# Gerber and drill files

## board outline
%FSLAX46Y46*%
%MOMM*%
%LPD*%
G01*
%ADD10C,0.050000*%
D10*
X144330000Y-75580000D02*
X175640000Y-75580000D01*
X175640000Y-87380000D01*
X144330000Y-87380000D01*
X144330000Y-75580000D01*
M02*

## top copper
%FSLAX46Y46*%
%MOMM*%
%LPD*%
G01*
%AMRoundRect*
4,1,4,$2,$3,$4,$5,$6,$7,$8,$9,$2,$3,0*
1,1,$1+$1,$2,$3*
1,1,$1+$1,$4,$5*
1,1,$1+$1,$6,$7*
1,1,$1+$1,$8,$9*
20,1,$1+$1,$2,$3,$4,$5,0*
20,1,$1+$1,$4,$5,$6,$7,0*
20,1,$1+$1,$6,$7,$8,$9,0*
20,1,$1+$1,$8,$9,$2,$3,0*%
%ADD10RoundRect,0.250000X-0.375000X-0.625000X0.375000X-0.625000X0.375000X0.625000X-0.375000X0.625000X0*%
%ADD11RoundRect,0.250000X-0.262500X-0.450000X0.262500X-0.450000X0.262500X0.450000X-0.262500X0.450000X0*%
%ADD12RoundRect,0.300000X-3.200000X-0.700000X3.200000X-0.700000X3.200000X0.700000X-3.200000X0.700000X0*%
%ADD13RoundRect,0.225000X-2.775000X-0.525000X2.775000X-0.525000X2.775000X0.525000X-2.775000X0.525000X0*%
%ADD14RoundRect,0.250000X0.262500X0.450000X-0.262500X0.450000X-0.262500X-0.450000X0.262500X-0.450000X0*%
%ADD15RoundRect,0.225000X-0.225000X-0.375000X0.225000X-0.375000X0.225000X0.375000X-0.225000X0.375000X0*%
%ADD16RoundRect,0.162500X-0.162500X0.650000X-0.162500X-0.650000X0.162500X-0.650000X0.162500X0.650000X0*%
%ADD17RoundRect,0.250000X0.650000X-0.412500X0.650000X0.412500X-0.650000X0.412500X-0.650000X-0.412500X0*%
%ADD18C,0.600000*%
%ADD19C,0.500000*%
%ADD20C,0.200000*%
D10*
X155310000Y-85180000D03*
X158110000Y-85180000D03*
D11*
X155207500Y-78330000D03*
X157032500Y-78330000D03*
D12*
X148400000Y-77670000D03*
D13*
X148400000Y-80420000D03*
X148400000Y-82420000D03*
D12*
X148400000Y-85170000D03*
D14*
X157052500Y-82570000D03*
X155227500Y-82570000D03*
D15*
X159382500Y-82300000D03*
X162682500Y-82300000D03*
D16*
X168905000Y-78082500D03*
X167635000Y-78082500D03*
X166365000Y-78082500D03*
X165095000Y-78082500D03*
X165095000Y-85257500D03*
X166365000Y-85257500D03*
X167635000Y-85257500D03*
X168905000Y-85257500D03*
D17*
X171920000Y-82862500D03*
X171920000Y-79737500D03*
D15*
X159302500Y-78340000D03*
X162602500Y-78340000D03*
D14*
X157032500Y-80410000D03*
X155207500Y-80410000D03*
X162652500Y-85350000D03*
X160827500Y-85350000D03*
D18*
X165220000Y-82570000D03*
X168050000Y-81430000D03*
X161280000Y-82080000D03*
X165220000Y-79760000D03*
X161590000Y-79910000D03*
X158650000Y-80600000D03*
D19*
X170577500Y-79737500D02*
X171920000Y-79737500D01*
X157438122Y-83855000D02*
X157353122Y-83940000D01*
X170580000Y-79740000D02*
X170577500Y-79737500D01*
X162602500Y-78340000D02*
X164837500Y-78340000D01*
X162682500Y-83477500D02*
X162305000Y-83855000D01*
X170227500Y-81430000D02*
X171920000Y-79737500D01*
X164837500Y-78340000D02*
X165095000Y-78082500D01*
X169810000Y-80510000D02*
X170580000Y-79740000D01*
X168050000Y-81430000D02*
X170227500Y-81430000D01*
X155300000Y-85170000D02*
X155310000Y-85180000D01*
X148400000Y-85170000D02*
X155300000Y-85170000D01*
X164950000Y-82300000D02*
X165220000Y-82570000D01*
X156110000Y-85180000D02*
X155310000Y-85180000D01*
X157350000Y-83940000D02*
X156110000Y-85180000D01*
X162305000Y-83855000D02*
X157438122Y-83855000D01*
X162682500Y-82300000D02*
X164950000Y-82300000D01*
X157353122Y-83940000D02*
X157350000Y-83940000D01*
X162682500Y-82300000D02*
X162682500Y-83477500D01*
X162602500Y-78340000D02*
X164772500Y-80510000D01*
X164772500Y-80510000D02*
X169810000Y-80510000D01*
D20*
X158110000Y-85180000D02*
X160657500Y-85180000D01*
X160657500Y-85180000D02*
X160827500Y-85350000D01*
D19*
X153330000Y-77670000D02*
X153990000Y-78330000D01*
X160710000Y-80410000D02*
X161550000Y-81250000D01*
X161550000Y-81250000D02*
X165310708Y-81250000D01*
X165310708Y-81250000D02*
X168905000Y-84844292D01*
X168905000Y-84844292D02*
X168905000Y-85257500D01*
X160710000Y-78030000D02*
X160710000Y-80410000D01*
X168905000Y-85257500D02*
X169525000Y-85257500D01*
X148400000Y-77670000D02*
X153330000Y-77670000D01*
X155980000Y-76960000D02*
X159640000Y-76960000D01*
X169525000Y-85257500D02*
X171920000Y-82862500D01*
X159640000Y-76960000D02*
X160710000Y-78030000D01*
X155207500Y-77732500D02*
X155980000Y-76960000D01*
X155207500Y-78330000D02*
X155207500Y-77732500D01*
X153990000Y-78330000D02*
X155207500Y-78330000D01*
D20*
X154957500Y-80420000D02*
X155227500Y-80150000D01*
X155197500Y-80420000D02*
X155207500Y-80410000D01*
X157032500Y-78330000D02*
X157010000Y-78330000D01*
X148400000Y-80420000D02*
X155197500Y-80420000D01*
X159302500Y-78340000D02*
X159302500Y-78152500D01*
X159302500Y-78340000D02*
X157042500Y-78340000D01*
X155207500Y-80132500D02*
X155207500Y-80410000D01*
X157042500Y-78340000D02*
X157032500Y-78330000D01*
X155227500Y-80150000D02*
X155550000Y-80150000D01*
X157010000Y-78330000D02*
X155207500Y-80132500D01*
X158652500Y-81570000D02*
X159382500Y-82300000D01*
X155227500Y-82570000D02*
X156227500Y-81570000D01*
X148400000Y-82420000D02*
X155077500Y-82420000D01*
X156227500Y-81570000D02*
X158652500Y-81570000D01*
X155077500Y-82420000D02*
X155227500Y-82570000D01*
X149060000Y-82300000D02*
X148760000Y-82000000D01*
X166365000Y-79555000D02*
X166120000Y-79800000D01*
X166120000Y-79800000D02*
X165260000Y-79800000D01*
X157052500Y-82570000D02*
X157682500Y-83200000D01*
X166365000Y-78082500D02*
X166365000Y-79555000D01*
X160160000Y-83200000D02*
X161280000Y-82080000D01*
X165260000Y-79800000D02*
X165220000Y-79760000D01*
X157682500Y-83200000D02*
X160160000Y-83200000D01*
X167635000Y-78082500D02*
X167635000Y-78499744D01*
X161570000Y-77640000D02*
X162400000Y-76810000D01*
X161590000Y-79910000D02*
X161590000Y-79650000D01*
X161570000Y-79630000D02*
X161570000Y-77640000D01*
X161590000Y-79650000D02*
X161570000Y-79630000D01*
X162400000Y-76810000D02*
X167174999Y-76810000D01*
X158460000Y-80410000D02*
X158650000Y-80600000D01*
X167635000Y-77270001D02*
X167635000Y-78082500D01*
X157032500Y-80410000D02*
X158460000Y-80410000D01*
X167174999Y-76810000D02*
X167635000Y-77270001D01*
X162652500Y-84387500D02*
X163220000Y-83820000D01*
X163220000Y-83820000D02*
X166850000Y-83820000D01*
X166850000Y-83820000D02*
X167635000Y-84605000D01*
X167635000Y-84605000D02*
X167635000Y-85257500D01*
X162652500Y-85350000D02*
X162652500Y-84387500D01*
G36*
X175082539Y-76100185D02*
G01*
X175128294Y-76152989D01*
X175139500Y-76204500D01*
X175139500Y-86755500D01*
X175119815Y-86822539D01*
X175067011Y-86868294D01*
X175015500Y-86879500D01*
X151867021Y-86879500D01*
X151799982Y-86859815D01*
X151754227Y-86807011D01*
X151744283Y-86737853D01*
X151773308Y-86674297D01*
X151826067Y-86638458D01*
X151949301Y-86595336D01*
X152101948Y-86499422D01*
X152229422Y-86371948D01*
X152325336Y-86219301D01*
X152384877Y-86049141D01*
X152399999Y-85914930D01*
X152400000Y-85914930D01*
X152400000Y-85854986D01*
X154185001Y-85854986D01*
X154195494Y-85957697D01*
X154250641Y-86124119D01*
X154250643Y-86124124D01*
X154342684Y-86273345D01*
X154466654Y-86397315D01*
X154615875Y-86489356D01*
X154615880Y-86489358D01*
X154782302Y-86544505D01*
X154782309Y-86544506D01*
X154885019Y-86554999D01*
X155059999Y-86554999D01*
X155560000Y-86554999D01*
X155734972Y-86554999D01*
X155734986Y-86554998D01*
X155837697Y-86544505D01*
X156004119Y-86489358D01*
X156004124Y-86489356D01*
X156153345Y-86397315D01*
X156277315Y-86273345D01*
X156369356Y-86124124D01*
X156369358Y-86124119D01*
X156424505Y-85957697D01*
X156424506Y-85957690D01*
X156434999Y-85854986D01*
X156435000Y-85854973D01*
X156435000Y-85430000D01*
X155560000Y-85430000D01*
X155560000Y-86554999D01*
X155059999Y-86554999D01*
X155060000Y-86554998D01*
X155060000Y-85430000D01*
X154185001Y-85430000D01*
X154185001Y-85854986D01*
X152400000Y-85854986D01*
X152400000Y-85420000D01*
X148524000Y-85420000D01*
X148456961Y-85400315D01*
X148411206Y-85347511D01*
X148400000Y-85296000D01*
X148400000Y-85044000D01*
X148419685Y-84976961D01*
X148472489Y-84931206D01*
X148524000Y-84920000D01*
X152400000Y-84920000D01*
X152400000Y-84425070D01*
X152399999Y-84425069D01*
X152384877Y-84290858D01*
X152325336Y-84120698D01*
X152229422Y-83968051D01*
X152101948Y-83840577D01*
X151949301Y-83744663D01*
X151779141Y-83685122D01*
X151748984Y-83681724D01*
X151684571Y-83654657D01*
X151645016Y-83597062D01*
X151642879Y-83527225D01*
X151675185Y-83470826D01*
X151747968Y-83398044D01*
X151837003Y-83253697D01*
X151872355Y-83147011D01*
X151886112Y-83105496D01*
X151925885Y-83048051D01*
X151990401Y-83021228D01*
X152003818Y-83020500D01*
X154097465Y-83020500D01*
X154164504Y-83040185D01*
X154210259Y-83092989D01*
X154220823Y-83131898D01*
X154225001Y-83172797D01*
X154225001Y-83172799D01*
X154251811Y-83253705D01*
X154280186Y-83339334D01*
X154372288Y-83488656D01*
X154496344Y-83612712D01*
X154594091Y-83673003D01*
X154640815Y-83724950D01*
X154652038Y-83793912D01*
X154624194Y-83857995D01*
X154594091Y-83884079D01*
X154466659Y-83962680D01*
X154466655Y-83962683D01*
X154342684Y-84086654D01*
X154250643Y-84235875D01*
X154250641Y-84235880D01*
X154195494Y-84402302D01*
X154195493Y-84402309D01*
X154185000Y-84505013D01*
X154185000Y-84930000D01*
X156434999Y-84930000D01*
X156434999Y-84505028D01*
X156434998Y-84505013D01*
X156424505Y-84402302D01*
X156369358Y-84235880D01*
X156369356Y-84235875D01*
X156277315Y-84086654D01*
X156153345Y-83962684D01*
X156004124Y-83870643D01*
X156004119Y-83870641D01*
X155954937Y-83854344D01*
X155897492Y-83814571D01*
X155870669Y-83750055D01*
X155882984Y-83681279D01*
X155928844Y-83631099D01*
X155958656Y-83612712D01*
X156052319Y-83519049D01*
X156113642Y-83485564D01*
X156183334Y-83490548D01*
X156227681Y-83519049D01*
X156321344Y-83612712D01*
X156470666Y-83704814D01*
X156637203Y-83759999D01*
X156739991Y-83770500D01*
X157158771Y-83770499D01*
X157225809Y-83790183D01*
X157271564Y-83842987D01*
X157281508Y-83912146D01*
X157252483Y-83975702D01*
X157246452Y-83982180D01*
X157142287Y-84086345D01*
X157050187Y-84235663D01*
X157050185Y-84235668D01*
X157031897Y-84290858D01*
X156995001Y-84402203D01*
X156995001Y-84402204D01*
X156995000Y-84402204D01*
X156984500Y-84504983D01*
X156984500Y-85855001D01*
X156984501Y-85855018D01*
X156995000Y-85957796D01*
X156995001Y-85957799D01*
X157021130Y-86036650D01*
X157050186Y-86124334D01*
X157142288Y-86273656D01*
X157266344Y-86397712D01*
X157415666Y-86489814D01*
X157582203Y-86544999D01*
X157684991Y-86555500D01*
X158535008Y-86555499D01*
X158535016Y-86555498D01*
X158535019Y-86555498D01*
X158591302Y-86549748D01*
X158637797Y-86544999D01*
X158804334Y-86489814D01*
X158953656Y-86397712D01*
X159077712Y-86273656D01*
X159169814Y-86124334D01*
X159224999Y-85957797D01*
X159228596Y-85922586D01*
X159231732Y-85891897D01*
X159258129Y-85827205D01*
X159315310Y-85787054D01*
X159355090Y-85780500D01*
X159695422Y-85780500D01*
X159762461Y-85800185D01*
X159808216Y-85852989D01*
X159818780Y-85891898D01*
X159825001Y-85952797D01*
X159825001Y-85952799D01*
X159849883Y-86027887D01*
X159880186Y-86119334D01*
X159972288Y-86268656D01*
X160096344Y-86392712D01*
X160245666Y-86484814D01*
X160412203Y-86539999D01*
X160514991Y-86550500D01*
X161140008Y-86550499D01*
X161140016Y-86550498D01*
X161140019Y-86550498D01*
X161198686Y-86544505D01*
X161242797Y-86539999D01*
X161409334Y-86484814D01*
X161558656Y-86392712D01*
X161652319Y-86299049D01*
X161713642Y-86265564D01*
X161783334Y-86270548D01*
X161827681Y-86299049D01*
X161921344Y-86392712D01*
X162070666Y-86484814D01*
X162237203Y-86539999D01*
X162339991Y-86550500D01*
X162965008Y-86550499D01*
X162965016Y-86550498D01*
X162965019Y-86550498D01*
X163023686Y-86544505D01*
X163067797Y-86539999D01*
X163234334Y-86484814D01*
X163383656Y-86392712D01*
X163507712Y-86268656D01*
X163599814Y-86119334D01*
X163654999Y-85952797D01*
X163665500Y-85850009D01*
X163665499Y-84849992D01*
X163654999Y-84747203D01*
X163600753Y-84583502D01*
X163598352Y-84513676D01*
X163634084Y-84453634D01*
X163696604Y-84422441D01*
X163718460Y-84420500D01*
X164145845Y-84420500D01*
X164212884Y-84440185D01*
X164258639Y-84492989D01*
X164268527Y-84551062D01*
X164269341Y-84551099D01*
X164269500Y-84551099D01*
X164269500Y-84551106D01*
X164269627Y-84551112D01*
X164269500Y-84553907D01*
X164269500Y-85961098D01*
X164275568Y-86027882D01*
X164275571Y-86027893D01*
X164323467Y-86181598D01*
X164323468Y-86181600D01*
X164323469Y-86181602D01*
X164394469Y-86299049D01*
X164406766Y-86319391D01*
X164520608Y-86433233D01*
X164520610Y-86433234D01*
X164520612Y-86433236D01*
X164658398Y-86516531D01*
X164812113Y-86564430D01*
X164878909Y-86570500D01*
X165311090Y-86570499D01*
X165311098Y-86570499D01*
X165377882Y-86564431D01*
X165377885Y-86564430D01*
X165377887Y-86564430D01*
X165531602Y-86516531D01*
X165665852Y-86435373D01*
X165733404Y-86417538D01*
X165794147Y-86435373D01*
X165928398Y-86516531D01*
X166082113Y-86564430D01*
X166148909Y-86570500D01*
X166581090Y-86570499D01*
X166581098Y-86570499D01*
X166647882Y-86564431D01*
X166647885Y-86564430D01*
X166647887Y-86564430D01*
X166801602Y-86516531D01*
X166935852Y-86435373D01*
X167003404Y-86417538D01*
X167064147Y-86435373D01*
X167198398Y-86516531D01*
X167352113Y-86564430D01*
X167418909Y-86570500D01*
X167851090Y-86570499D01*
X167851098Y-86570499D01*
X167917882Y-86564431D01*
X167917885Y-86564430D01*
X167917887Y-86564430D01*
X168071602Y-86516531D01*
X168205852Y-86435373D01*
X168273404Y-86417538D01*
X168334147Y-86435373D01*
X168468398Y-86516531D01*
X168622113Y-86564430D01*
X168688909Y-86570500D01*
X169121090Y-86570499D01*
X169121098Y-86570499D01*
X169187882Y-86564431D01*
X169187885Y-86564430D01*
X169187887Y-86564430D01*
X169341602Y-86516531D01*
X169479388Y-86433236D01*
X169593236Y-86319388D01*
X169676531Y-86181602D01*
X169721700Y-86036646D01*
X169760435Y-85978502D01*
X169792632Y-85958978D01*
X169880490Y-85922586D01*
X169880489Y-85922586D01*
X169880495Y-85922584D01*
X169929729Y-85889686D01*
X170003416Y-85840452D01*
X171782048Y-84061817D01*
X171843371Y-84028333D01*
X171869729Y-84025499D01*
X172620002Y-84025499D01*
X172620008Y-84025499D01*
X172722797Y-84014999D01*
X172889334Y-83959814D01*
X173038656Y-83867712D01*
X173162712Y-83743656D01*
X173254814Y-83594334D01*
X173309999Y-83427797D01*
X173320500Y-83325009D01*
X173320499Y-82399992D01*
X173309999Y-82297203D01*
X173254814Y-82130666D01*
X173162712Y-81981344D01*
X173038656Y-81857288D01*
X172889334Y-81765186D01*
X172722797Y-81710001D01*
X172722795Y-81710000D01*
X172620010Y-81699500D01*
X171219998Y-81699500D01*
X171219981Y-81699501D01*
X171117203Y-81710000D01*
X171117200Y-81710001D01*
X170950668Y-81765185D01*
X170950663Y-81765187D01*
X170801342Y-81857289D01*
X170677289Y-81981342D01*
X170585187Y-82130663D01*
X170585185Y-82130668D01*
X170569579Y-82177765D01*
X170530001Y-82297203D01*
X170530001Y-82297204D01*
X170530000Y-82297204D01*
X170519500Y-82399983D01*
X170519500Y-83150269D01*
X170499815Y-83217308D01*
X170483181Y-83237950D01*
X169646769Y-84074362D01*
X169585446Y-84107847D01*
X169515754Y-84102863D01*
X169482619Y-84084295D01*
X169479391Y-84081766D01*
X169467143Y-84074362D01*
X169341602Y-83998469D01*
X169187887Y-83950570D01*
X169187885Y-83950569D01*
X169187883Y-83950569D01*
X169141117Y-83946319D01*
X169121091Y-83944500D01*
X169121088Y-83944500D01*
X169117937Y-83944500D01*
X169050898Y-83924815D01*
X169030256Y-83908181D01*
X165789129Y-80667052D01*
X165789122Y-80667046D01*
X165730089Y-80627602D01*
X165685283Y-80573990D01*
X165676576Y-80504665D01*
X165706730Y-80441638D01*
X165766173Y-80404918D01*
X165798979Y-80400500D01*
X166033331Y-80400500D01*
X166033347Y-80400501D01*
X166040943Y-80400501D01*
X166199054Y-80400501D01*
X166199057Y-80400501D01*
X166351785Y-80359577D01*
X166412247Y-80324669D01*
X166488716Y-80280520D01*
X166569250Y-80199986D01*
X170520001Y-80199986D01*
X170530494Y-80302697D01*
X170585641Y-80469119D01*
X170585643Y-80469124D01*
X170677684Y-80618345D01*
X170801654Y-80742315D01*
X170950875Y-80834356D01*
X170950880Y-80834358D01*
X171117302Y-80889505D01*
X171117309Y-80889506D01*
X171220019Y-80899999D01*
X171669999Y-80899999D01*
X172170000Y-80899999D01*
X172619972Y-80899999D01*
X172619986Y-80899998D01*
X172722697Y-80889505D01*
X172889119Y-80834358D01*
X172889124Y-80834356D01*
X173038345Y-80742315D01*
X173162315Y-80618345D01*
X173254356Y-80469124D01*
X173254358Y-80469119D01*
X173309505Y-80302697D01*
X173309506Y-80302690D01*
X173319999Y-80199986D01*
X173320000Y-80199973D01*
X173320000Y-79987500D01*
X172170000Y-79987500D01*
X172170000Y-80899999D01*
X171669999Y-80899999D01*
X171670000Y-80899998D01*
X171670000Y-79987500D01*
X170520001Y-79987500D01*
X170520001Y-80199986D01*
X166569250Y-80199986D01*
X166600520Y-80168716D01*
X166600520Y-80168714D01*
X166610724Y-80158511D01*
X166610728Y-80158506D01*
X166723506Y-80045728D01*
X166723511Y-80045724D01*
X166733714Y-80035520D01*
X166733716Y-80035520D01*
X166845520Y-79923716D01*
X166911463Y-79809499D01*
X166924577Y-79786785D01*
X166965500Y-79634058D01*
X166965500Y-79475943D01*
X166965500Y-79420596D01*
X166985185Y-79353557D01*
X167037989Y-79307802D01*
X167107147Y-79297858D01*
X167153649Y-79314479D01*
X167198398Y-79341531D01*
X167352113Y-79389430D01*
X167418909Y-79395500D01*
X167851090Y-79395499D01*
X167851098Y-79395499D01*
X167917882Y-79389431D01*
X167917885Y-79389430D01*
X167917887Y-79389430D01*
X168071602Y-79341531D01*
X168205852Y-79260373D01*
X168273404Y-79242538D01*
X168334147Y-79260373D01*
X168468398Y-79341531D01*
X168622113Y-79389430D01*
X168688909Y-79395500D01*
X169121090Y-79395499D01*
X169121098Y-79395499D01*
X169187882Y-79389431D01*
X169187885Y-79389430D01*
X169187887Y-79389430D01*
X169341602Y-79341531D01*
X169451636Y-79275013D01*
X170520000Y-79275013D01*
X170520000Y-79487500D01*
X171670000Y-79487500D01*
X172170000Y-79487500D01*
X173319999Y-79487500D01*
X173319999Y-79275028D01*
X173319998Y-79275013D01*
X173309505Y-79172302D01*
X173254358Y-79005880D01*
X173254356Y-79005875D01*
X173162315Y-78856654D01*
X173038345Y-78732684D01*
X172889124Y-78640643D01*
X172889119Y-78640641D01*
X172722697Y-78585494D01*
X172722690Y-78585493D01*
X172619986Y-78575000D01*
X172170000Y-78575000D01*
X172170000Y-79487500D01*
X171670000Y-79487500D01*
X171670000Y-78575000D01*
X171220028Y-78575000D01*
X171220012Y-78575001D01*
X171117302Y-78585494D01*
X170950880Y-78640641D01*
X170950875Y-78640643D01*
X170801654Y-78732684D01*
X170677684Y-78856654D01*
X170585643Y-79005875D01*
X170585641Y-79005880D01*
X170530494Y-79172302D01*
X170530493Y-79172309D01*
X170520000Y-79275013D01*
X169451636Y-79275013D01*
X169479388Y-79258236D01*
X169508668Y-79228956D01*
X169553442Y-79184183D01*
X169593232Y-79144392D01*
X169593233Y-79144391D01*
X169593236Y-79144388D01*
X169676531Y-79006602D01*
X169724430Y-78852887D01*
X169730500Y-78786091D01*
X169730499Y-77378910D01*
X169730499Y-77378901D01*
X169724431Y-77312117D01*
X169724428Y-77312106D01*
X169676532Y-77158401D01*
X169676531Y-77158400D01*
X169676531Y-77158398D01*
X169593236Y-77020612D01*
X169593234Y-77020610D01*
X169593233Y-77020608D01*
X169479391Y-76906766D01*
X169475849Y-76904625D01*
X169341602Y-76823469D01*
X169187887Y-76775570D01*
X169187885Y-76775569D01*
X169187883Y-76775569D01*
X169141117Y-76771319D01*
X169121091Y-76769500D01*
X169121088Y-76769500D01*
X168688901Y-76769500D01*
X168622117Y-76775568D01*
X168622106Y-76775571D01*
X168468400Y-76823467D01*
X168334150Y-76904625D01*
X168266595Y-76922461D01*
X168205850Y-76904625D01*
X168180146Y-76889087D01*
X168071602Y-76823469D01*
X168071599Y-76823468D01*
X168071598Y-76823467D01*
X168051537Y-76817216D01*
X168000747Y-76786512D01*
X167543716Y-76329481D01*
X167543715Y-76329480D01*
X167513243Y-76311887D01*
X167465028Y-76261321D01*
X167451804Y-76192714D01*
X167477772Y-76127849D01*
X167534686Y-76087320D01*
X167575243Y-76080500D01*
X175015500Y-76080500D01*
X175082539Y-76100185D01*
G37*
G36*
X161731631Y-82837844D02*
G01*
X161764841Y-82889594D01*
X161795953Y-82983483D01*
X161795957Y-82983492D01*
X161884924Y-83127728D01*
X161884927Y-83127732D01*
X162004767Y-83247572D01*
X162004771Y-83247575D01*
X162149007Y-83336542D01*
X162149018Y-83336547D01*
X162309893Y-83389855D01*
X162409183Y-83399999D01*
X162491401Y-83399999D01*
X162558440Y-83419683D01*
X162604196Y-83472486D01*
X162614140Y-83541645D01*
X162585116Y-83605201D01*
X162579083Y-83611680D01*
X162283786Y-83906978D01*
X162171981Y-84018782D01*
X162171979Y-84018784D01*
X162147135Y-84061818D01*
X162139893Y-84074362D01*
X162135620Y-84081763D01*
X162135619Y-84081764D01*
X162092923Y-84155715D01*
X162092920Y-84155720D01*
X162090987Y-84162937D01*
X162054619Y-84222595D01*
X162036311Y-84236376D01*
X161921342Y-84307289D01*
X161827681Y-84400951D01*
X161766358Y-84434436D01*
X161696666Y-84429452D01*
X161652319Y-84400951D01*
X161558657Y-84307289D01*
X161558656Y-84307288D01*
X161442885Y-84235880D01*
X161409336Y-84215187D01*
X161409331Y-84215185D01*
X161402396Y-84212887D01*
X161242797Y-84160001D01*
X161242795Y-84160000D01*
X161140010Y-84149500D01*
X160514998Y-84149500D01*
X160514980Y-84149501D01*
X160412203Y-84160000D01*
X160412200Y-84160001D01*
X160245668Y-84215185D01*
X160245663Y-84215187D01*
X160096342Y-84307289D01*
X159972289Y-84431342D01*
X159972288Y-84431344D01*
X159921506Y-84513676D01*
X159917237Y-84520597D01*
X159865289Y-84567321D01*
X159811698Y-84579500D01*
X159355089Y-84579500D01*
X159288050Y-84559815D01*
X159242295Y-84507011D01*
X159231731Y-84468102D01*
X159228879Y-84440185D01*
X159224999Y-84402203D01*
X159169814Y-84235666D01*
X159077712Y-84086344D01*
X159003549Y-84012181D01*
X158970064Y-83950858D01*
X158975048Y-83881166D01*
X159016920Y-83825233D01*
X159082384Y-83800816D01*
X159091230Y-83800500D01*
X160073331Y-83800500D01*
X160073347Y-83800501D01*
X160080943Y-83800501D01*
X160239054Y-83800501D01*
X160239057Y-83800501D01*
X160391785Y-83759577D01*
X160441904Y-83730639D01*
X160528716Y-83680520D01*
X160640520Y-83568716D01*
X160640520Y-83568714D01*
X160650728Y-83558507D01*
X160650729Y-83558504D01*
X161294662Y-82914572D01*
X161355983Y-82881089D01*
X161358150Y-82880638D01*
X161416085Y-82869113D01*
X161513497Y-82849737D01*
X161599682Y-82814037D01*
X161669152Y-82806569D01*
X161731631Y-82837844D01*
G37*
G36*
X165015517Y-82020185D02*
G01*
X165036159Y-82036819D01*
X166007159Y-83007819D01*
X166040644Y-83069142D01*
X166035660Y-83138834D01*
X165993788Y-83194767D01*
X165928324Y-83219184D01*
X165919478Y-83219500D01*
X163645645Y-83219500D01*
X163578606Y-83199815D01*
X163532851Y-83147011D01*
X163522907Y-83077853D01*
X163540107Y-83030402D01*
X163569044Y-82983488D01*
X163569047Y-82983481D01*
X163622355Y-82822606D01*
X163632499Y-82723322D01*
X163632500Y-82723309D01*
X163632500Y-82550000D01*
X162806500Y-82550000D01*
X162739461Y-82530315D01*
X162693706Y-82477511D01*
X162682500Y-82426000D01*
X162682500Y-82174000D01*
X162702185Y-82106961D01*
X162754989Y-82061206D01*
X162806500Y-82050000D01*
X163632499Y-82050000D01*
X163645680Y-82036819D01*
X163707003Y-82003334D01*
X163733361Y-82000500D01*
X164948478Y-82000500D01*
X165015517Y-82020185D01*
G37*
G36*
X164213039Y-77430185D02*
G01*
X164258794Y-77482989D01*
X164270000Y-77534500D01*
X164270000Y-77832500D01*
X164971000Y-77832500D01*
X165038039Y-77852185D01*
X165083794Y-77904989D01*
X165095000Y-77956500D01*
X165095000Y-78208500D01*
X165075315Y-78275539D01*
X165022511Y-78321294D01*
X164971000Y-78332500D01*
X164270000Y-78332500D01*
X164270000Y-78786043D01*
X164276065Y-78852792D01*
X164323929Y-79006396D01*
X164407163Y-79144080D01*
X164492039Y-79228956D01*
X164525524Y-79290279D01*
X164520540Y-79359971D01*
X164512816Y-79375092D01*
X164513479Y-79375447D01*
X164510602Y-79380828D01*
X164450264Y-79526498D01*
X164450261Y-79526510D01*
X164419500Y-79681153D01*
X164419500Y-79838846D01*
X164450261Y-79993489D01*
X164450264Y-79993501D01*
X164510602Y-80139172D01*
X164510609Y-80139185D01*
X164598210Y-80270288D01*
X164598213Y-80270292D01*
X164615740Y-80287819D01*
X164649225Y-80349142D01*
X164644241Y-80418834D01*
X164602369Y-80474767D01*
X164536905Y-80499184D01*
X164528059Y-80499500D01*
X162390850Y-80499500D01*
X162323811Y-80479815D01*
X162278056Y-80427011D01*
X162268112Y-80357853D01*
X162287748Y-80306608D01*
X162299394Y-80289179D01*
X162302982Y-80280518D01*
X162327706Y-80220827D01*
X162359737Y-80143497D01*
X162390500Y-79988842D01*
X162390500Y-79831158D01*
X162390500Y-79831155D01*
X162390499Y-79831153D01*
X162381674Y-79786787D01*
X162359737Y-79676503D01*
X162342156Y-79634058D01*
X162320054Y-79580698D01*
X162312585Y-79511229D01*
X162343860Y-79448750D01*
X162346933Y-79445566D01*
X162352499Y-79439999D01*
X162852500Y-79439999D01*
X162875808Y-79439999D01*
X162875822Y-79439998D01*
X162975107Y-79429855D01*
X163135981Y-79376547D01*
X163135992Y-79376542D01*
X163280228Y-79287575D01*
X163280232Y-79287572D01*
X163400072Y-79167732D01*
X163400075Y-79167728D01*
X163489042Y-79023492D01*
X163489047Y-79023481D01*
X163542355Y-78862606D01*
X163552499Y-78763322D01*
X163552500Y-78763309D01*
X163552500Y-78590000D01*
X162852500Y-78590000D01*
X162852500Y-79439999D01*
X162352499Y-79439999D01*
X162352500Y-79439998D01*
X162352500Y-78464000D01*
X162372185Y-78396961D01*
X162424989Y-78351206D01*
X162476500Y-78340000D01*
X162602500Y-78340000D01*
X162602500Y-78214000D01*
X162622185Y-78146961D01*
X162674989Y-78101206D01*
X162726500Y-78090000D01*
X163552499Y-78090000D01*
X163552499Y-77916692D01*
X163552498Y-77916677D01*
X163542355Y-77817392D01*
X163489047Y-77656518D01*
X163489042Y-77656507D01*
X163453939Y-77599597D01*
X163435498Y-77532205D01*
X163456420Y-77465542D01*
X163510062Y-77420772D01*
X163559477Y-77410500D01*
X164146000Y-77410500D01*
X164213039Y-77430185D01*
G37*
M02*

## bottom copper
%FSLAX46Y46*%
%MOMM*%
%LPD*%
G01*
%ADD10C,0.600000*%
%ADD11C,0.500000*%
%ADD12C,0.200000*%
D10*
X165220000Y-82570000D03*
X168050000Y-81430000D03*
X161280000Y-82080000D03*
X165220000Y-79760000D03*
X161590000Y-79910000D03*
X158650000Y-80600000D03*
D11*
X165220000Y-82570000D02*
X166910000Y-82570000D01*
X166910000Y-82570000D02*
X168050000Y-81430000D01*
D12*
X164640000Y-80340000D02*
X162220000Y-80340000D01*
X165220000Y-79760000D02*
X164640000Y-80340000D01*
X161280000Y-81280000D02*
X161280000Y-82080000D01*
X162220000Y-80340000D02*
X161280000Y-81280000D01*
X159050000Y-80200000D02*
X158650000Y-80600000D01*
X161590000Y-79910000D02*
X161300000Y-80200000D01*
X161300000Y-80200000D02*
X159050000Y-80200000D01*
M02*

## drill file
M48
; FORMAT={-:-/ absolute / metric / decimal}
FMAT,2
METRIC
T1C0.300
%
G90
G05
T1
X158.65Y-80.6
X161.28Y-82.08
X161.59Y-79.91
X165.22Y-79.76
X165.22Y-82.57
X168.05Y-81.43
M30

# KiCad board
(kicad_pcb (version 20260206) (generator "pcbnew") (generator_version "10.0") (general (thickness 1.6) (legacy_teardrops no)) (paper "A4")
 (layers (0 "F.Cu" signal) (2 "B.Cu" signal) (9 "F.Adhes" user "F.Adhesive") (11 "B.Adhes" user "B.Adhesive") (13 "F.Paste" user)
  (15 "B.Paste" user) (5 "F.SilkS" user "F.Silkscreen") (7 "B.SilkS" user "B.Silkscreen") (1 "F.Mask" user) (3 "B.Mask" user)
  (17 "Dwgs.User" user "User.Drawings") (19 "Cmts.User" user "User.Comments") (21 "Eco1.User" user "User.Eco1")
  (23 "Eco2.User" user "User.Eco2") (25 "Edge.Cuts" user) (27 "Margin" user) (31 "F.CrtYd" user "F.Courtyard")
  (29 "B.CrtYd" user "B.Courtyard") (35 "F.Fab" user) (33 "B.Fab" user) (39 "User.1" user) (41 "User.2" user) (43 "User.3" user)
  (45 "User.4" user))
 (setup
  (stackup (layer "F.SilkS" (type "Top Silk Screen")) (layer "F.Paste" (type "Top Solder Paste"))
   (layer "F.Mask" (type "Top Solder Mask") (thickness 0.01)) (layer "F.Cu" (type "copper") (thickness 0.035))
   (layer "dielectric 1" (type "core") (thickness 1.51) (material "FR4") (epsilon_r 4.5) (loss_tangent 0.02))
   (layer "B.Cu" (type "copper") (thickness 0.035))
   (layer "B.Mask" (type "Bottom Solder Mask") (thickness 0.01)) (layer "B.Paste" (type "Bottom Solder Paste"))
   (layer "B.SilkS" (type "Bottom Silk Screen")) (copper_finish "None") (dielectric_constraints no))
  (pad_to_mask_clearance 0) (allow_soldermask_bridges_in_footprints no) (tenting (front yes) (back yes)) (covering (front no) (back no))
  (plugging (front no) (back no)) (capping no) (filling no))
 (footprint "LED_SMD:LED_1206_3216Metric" (layer "F.Cu") (at 156.71 85.18)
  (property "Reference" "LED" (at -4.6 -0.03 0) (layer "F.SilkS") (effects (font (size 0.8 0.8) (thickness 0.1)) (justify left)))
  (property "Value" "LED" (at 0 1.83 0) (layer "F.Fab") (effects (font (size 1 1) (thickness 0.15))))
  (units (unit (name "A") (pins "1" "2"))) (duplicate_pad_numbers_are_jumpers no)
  (pad "1" smd roundrect (at -1.4 0) (size 1.25 1.75) (layers "F.Cu" "F.Mask" "F.Paste") (roundrect_rratio 0.2) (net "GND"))
  (pad "2" smd roundrect (at 1.4 0) (size 1.25 1.75) (layers "F.Cu" "F.Mask" "F.Paste") (roundrect_rratio 0.2) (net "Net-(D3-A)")))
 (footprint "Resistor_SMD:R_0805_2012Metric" (layer "F.Cu") (at 156.12 78.33)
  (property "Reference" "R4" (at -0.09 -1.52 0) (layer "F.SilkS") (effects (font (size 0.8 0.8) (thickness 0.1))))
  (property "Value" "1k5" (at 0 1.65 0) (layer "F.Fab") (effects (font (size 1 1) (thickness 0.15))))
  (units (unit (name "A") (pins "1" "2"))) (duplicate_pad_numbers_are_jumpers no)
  (pad "1" smd roundrect (at -0.9125 0) (size 1.025 1.4) (layers "F.Cu" "F.Mask" "F.Paste") (roundrect_rratio 0.243902) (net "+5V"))
  (pad "2" smd roundrect (at 0.9125 0) (size 1.025 1.4) (layers "F.Cu" "F.Mask" "F.Paste") (roundrect_rratio 0.243902) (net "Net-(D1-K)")))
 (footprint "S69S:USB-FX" (layer "F.Cu") (at 148.4 81.42)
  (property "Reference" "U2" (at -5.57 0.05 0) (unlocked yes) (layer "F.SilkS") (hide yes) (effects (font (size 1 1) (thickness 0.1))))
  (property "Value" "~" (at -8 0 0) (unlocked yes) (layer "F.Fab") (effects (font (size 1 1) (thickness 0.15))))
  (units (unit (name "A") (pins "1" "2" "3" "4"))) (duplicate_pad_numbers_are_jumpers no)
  (pad "1" smd roundrect (at 0 -3.75) (size 7 2) (layers "F.Cu" "F.Mask" "F.Paste") (roundrect_rratio 0.15) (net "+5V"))
  (pad "2" smd roundrect (at 0 -1) (size 6 1.5) (layers "F.Cu" "F.Mask" "F.Paste") (roundrect_rratio 0.15) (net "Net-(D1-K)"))
  (pad "3" smd roundrect (at 0 1) (size 6 1.5) (layers "F.Cu" "F.Mask" "F.Paste") (roundrect_rratio 0.15) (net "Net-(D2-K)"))
  (pad "4" smd roundrect (at 0 3.75) (size 7 2) (layers "F.Cu" "F.Mask" "F.Paste") (roundrect_rratio 0.15) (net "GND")))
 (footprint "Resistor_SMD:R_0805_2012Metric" (layer "F.Cu") (at 156.14 82.57 180)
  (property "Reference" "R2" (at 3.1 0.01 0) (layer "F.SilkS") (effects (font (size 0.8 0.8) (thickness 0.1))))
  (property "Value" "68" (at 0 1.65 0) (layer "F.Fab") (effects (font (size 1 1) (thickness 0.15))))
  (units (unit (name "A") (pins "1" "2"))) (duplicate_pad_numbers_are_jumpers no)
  (pad "1" smd roundrect (at -0.9125 0 180) (size 1.025 1.4) (layers "F.Cu" "F.Mask" "F.Paste") (roundrect_rratio 0.243902)
   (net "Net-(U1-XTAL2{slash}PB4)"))
  (pad "2" smd roundrect (at 0.9125 0 180) (size 1.025 1.4) (layers "F.Cu" "F.Mask" "F.Paste") (roundrect_rratio 0.243902)
   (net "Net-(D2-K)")))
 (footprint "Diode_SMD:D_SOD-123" (layer "F.Cu") (at 161.0325 82.3)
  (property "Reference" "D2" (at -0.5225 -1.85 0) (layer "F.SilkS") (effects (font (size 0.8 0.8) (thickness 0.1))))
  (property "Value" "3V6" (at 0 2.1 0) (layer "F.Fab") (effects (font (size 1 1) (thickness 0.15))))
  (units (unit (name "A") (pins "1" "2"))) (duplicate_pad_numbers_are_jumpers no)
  (pad "1" smd roundrect (at -1.65 0) (size 0.9 1.2) (layers "F.Cu" "F.Mask" "F.Paste") (roundrect_rratio 0.25) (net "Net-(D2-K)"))
  (pad "2" smd roundrect (at 1.65 0) (size 0.9 1.2) (layers "F.Cu" "F.Mask" "F.Paste") (roundrect_rratio 0.25) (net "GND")))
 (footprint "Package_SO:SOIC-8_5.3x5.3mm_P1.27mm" (layer "F.Cu") (at 167 81.67 -90)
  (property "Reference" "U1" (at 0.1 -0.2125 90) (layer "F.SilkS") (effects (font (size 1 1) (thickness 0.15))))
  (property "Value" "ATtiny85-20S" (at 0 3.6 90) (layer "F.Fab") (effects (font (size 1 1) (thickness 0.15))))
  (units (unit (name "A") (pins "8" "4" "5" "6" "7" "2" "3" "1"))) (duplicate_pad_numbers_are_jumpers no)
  (pad "1" smd roundrect (at -3.5875 -1.905 270) (size 1.625 0.65) (layers "F.Cu" "F.Mask" "F.Paste") (roundrect_rratio 0.25)
   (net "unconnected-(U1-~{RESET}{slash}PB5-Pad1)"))
  (pad "2" smd roundrect (at -3.5875 -0.635 270) (size 1.625 0.65) (layers "F.Cu" "F.Mask" "F.Paste") (roundrect_rratio 0.25)
   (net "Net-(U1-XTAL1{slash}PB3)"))
  (pad "3" smd roundrect (at -3.5875 0.635 270) (size 1.625 0.65) (layers "F.Cu" "F.Mask" "F.Paste") (roundrect_rratio 0.25)
   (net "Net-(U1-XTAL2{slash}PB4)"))
  (pad "4" smd roundrect (at -3.5875 1.905 270) (size 1.625 0.65) (layers "F.Cu" "F.Mask" "F.Paste") (roundrect_rratio 0.25) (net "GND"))
  (pad "5" smd roundrect (at 3.5875 1.905 270) (size 1.625 0.65) (layers "F.Cu" "F.Mask" "F.Paste") (roundrect_rratio 0.25)
   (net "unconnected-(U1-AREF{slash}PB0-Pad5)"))
  (pad "6" smd roundrect (at 3.5875 0.635 270) (size 1.625 0.65) (layers "F.Cu" "F.Mask" "F.Paste") (roundrect_rratio 0.25)
   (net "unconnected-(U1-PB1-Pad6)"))
  (pad "7" smd roundrect (at 3.5875 -0.635 270) (size 1.625 0.65) (layers "F.Cu" "F.Mask" "F.Paste") (roundrect_rratio 0.25)
   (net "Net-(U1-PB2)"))
  (pad "8" smd roundrect (at 3.5875 -1.905 270) (size 1.625 0.65) (layers "F.Cu" "F.Mask" "F.Paste") (roundrect_rratio 0.25) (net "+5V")))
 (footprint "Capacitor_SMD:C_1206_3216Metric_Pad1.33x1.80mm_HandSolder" (layer "F.Cu") (at 171.92 81.3 90)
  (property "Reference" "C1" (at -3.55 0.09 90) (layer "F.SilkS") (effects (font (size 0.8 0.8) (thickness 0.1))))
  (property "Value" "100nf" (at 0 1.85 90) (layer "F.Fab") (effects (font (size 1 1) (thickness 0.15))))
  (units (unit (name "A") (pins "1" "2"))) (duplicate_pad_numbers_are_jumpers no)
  (pad "1" smd roundrect (at -1.5625 0 90) (size 1.325 1.8) (layers "F.Cu" "F.Mask" "F.Paste") (roundrect_rratio 0.188679) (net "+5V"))
  (pad "2" smd roundrect (at 1.5625 0 90) (size 1.325 1.8) (layers "F.Cu" "F.Mask" "F.Paste") (roundrect_rratio 0.188679) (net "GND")))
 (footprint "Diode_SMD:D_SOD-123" (layer "F.Cu") (at 160.9525 78.34)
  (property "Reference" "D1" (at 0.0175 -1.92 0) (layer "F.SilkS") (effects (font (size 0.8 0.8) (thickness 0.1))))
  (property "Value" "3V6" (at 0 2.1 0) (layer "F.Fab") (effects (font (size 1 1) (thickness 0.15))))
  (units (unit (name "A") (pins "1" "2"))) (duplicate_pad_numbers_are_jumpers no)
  (pad "1" smd roundrect (at -1.65 0) (size 0.9 1.2) (layers "F.Cu" "F.Mask" "F.Paste") (roundrect_rratio 0.25) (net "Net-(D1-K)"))
  (pad "2" smd roundrect (at 1.65 0) (size 0.9 1.2) (layers "F.Cu" "F.Mask" "F.Paste") (roundrect_rratio 0.25) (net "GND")))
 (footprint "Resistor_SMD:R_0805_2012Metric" (layer "F.Cu") (at 156.12 80.41 180)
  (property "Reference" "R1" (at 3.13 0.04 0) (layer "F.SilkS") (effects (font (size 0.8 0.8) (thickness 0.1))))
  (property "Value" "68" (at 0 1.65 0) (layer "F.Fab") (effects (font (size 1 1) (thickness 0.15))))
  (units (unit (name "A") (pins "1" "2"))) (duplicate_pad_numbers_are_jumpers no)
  (pad "1" smd roundrect (at -0.9125 0 180) (size 1.025 1.4) (layers "F.Cu" "F.Mask" "F.Paste") (roundrect_rratio 0.243902)
   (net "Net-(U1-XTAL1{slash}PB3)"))
  (pad "2" smd roundrect (at 0.9125 0 180) (size 1.025 1.4) (layers "F.Cu" "F.Mask" "F.Paste") (roundrect_rratio 0.243902)
   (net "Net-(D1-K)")))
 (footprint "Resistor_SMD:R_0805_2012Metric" (layer "F.Cu") (at 161.74 85.35 180)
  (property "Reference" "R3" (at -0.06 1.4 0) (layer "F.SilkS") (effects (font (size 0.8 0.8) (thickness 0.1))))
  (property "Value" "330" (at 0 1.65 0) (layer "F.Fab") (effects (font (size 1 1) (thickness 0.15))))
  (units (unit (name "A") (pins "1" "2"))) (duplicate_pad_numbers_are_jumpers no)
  (pad "1" smd roundrect (at -0.9125 0 180) (size 1.025 1.4) (layers "F.Cu" "F.Mask" "F.Paste") (roundrect_rratio 0.243902)
   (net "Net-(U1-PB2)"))
  (pad "2" smd roundrect (at 0.9125 0 180) (size 1.025 1.4) (layers "F.Cu" "F.Mask" "F.Paste") (roundrect_rratio 0.243902)
   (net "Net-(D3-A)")))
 (gr_rect (start 144.33 75.58) (end 175.64 87.38) (stroke (width 0.05) (type solid)) (fill no) (layer "Edge.Cuts"))
 (segment (start 170.5775 79.7375) (end 171.92 79.7375) (width 0.5) (layer "F.Cu") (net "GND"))
 (segment (start 157.438122 83.855) (end 157.353122 83.94) (width 0.5) (layer "F.Cu") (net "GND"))
 (segment (start 170.58 79.74) (end 170.5775 79.7375) (width 0.5) (layer "F.Cu") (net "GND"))
 (segment (start 162.6025 78.34) (end 164.8375 78.34) (width 0.5) (layer "F.Cu") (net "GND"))
 (segment (start 162.6825 83.4775) (end 162.305 83.855) (width 0.5) (layer "F.Cu") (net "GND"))
 (segment (start 170.2275 81.43) (end 171.92 79.7375) (width 0.5) (layer "F.Cu") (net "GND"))
 (segment (start 164.8375 78.34) (end 165.095 78.0825) (width 0.5) (layer "F.Cu") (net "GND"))
 (segment (start 169.81 80.51) (end 170.58 79.74) (width 0.5) (layer "F.Cu") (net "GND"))
 (segment (start 168.05 81.43) (end 170.2275 81.43) (width 0.5) (layer "F.Cu") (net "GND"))
 (segment (start 155.3 85.17) (end 155.31 85.18) (width 0.5) (layer "F.Cu") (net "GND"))
 (segment (start 148.4 85.17) (end 155.3 85.17) (width 0.5) (layer "F.Cu") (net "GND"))
 (segment (start 164.95 82.3) (end 165.22 82.57) (width 0.5) (layer "F.Cu") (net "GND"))
 (segment (start 156.11 85.18) (end 155.31 85.18) (width 0.5) (layer "F.Cu") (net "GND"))
 (segment (start 157.35 83.94) (end 156.11 85.18) (width 0.5) (layer "F.Cu") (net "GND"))
 (segment (start 162.305 83.855) (end 157.438122 83.855) (width 0.5) (layer "F.Cu") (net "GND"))
 (segment (start 162.6825 82.3) (end 164.95 82.3) (width 0.5) (layer "F.Cu") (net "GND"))
 (segment (start 157.353122 83.94) (end 157.35 83.94) (width 0.5) (layer "F.Cu") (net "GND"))
 (segment (start 162.6825 82.3) (end 162.6825 83.4775) (width 0.5) (layer "F.Cu") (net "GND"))
 (segment (start 162.6025 78.34) (end 164.7725 80.51) (width 0.5) (layer "F.Cu") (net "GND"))
 (segment (start 164.7725 80.51) (end 169.81 80.51) (width 0.5) (layer "F.Cu") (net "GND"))
 (via (at 165.22 82.57) (size 0.6) (drill 0.3) (layers "F.Cu" "B.Cu") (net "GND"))
 (via (at 168.05 81.43) (size 0.6) (drill 0.3) (layers "F.Cu" "B.Cu") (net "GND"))
 (segment (start 165.22 82.57) (end 166.91 82.57) (width 0.5) (layer "B.Cu") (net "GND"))
 (segment (start 166.91 82.57) (end 168.05 81.43) (width 0.5) (layer "B.Cu") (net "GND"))
 (segment (start 158.11 85.18) (end 160.6575 85.18) (width 0.2) (layer "F.Cu") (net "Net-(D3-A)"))
 (segment (start 160.6575 85.18) (end 160.8275 85.35) (width 0.2) (layer "F.Cu") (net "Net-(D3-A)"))
 (segment (start 153.33 77.67) (end 153.99 78.33) (width 0.5) (layer "F.Cu") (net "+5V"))
 (segment (start 160.71 80.41) (end 161.55 81.25) (width 0.5) (layer "F.Cu") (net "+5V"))
 (segment (start 161.55 81.25) (end 165.310708 81.25) (width 0.5) (layer "F.Cu") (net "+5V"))
 (segment (start 165.310708 81.25) (end 168.905 84.844292) (width 0.5) (layer "F.Cu") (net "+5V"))
 (segment (start 168.905 84.844292) (end 168.905 85.2575) (width 0.5) (layer "F.Cu") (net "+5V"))
 (segment (start 160.71 78.03) (end 160.71 80.41) (width 0.5) (layer "F.Cu") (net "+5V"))
 (segment (start 168.905 85.2575) (end 169.525 85.2575) (width 0.5) (layer "F.Cu") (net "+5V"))
 (segment (start 148.4 77.67) (end 153.33 77.67) (width 0.5) (layer "F.Cu") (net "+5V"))
 (segment (start 155.98 76.96) (end 159.64 76.96) (width 0.5) (layer "F.Cu") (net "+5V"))
 (segment (start 169.525 85.2575) (end 171.92 82.8625) (width 0.5) (layer "F.Cu") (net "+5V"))
 (segment (start 159.64 76.96) (end 160.71 78.03) (width 0.5) (layer "F.Cu") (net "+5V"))
 (segment (start 155.2075 77.7325) (end 155.98 76.96) (width 0.5) (layer "F.Cu") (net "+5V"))
 (segment (start 155.2075 78.33) (end 155.2075 77.7325) (width 0.5) (layer "F.Cu") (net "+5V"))
 (segment (start 153.99 78.33) (end 155.2075 78.33) (width 0.5) (layer "F.Cu") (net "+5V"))
 (segment (start 154.9575 80.42) (end 155.2275 80.15) (width 0.2) (layer "F.Cu") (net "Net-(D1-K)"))
 (segment (start 155.1975 80.42) (end 155.2075 80.41) (width 0.2) (layer "F.Cu") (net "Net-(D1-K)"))
 (segment (start 157.0325 78.33) (end 157.01 78.33) (width 0.2) (layer "F.Cu") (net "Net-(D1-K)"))
 (segment (start 148.4 80.42) (end 155.1975 80.42) (width 0.2) (layer "F.Cu") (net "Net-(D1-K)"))
 (segment (start 159.3025 78.34) (end 159.3025 78.1525) (width 0.2) (layer "F.Cu") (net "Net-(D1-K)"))
 (segment (start 159.3025 78.34) (end 157.0425 78.34) (width 0.2) (layer "F.Cu") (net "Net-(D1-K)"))
 (segment (start 155.2075 80.1325) (end 155.2075 80.41) (width 0.2) (layer "F.Cu") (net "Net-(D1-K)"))
 (segment (start 157.0425 78.34) (end 157.0325 78.33) (width 0.2) (layer "F.Cu") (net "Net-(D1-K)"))
 (segment (start 155.2275 80.15) (end 155.55 80.15) (width 0.2) (layer "F.Cu") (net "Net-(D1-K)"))
 (segment (start 157.01 78.33) (end 155.2075 80.1325) (width 0.2) (layer "F.Cu") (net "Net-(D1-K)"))
 (segment (start 158.6525 81.57) (end 159.3825 82.3) (width 0.2) (layer "F.Cu") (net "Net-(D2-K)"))
 (segment (start 155.2275 82.57) (end 156.2275 81.57) (width 0.2) (layer "F.Cu") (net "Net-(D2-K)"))
 (segment (start 148.4 82.42) (end 155.0775 82.42) (width 0.2) (layer "F.Cu") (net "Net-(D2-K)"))
 (segment (start 156.2275 81.57) (end 158.6525 81.57) (width 0.2) (layer "F.Cu") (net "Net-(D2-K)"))
 (segment (start 155.0775 82.42) (end 155.2275 82.57) (width 0.2) (layer "F.Cu") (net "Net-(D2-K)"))
 (segment (start 149.06 82.3) (end 148.76 82) (width 0.2) (layer "F.Cu") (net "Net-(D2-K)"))
 (segment (start 166.365 79.555) (end 166.12 79.8) (width 0.2) (layer "F.Cu") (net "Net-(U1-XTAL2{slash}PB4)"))
 (segment (start 166.12 79.8) (end 165.26 79.8) (width 0.2) (layer "F.Cu") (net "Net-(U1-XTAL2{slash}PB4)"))
 (segment (start 157.0525 82.57) (end 157.6825 83.2) (width 0.2) (layer "F.Cu") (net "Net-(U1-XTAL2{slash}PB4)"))
 (segment (start 166.365 78.0825) (end 166.365 79.555) (width 0.2) (layer "F.Cu") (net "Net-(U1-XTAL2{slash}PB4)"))
 (segment (start 160.16 83.2) (end 161.28 82.08) (width 0.2) (layer "F.Cu") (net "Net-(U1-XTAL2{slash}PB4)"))
 (segment (start 165.26 79.8) (end 165.22 79.76) (width 0.2) (layer "F.Cu") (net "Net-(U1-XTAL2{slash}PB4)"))
 (segment (start 157.6825 83.2) (end 160.16 83.2) (width 0.2) (layer "F.Cu") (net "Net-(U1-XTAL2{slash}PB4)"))
 (via (at 161.28 82.08) (size 0.6) (drill 0.3) (layers "F.Cu" "B.Cu") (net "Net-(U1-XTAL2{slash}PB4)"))
 (via (at 165.22 79.76) (size 0.6) (drill 0.3) (layers "F.Cu" "B.Cu") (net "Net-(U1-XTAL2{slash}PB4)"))
 (segment (start 164.64 80.34) (end 162.22 80.34) (width 0.2) (layer "B.Cu") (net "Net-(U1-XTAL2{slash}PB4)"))
 (segment (start 165.22 79.76) (end 164.64 80.34) (width 0.2) (layer "B.Cu") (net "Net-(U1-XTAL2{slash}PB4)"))
 (segment (start 161.28 81.28) (end 161.28 82.08) (width 0.2) (layer "B.Cu") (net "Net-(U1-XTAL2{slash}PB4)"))
 (segment (start 162.22 80.34) (end 161.28 81.28) (width 0.2) (layer "B.Cu") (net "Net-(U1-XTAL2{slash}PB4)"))
 (segment (start 167.635 78.0825) (end 167.635 78.499744) (width 0.2) (layer "F.Cu") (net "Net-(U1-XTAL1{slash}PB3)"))
 (segment (start 161.57 77.64) (end 162.4 76.81) (width 0.2) (layer "F.Cu") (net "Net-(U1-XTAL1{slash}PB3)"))
 (segment (start 161.59 79.91) (end 161.59 79.65) (width 0.2) (layer "F.Cu") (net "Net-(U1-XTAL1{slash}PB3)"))
 (segment (start 161.57 79.63) (end 161.57 77.64) (width 0.2) (layer "F.Cu") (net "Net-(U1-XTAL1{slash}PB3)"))
 (segment (start 161.59 79.65) (end 161.57 79.63) (width 0.2) (layer "F.Cu") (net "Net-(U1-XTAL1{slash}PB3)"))
 (segment (start 162.4 76.81) (end 167.174999 76.81) (width 0.2) (layer "F.Cu") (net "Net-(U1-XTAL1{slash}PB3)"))
 (segment (start 158.46 80.41) (end 158.65 80.6) (width 0.2) (layer "F.Cu") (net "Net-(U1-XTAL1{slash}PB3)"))
 (segment (start 167.635 77.270001) (end 167.635 78.0825) (width 0.2) (layer "F.Cu") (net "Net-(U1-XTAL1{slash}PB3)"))
 (segment (start 157.0325 80.41) (end 158.46 80.41) (width 0.2) (layer "F.Cu") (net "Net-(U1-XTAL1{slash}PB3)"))
 (segment (start 167.174999 76.81) (end 167.635 77.270001) (width 0.2) (layer "F.Cu") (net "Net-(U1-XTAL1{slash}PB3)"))
 (via (at 161.59 79.91) (size 0.6) (drill 0.3) (layers "F.Cu" "B.Cu") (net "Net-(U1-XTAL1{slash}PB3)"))
 (via (at 158.65 80.6) (size 0.6) (drill 0.3) (layers "F.Cu" "B.Cu") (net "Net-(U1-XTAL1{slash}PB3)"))
 (segment (start 159.05 80.2) (end 158.65 80.6) (width 0.2) (layer "B.Cu") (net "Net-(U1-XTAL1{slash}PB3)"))
 (segment (start 161.59 79.91) (end 161.3 80.2) (width 0.2) (layer "B.Cu") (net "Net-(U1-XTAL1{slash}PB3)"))
 (segment (start 161.3 80.2) (end 159.05 80.2) (width 0.2) (layer "B.Cu") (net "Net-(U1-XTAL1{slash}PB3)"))
 (segment (start 162.6525 84.3875) (end 163.22 83.82) (width 0.2) (layer "F.Cu") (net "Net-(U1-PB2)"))
 (segment (start 163.22 83.82) (end 166.85 83.82) (width 0.2) (layer "F.Cu") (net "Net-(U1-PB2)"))
 (segment (start 166.85 83.82) (end 167.635 84.605) (width 0.2) (layer "F.Cu") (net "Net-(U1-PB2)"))
 (segment (start 167.635 84.605) (end 167.635 85.2575) (width 0.2) (layer "F.Cu") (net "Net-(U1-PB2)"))
 (segment (start 162.6525 85.35) (end 162.6525 84.3875) (width 0.2) (layer "F.Cu") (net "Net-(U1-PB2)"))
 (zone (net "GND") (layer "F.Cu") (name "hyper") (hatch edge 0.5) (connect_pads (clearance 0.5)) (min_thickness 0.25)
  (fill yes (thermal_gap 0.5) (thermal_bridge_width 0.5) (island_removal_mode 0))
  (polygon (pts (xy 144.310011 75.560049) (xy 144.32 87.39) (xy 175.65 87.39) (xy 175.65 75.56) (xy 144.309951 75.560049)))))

